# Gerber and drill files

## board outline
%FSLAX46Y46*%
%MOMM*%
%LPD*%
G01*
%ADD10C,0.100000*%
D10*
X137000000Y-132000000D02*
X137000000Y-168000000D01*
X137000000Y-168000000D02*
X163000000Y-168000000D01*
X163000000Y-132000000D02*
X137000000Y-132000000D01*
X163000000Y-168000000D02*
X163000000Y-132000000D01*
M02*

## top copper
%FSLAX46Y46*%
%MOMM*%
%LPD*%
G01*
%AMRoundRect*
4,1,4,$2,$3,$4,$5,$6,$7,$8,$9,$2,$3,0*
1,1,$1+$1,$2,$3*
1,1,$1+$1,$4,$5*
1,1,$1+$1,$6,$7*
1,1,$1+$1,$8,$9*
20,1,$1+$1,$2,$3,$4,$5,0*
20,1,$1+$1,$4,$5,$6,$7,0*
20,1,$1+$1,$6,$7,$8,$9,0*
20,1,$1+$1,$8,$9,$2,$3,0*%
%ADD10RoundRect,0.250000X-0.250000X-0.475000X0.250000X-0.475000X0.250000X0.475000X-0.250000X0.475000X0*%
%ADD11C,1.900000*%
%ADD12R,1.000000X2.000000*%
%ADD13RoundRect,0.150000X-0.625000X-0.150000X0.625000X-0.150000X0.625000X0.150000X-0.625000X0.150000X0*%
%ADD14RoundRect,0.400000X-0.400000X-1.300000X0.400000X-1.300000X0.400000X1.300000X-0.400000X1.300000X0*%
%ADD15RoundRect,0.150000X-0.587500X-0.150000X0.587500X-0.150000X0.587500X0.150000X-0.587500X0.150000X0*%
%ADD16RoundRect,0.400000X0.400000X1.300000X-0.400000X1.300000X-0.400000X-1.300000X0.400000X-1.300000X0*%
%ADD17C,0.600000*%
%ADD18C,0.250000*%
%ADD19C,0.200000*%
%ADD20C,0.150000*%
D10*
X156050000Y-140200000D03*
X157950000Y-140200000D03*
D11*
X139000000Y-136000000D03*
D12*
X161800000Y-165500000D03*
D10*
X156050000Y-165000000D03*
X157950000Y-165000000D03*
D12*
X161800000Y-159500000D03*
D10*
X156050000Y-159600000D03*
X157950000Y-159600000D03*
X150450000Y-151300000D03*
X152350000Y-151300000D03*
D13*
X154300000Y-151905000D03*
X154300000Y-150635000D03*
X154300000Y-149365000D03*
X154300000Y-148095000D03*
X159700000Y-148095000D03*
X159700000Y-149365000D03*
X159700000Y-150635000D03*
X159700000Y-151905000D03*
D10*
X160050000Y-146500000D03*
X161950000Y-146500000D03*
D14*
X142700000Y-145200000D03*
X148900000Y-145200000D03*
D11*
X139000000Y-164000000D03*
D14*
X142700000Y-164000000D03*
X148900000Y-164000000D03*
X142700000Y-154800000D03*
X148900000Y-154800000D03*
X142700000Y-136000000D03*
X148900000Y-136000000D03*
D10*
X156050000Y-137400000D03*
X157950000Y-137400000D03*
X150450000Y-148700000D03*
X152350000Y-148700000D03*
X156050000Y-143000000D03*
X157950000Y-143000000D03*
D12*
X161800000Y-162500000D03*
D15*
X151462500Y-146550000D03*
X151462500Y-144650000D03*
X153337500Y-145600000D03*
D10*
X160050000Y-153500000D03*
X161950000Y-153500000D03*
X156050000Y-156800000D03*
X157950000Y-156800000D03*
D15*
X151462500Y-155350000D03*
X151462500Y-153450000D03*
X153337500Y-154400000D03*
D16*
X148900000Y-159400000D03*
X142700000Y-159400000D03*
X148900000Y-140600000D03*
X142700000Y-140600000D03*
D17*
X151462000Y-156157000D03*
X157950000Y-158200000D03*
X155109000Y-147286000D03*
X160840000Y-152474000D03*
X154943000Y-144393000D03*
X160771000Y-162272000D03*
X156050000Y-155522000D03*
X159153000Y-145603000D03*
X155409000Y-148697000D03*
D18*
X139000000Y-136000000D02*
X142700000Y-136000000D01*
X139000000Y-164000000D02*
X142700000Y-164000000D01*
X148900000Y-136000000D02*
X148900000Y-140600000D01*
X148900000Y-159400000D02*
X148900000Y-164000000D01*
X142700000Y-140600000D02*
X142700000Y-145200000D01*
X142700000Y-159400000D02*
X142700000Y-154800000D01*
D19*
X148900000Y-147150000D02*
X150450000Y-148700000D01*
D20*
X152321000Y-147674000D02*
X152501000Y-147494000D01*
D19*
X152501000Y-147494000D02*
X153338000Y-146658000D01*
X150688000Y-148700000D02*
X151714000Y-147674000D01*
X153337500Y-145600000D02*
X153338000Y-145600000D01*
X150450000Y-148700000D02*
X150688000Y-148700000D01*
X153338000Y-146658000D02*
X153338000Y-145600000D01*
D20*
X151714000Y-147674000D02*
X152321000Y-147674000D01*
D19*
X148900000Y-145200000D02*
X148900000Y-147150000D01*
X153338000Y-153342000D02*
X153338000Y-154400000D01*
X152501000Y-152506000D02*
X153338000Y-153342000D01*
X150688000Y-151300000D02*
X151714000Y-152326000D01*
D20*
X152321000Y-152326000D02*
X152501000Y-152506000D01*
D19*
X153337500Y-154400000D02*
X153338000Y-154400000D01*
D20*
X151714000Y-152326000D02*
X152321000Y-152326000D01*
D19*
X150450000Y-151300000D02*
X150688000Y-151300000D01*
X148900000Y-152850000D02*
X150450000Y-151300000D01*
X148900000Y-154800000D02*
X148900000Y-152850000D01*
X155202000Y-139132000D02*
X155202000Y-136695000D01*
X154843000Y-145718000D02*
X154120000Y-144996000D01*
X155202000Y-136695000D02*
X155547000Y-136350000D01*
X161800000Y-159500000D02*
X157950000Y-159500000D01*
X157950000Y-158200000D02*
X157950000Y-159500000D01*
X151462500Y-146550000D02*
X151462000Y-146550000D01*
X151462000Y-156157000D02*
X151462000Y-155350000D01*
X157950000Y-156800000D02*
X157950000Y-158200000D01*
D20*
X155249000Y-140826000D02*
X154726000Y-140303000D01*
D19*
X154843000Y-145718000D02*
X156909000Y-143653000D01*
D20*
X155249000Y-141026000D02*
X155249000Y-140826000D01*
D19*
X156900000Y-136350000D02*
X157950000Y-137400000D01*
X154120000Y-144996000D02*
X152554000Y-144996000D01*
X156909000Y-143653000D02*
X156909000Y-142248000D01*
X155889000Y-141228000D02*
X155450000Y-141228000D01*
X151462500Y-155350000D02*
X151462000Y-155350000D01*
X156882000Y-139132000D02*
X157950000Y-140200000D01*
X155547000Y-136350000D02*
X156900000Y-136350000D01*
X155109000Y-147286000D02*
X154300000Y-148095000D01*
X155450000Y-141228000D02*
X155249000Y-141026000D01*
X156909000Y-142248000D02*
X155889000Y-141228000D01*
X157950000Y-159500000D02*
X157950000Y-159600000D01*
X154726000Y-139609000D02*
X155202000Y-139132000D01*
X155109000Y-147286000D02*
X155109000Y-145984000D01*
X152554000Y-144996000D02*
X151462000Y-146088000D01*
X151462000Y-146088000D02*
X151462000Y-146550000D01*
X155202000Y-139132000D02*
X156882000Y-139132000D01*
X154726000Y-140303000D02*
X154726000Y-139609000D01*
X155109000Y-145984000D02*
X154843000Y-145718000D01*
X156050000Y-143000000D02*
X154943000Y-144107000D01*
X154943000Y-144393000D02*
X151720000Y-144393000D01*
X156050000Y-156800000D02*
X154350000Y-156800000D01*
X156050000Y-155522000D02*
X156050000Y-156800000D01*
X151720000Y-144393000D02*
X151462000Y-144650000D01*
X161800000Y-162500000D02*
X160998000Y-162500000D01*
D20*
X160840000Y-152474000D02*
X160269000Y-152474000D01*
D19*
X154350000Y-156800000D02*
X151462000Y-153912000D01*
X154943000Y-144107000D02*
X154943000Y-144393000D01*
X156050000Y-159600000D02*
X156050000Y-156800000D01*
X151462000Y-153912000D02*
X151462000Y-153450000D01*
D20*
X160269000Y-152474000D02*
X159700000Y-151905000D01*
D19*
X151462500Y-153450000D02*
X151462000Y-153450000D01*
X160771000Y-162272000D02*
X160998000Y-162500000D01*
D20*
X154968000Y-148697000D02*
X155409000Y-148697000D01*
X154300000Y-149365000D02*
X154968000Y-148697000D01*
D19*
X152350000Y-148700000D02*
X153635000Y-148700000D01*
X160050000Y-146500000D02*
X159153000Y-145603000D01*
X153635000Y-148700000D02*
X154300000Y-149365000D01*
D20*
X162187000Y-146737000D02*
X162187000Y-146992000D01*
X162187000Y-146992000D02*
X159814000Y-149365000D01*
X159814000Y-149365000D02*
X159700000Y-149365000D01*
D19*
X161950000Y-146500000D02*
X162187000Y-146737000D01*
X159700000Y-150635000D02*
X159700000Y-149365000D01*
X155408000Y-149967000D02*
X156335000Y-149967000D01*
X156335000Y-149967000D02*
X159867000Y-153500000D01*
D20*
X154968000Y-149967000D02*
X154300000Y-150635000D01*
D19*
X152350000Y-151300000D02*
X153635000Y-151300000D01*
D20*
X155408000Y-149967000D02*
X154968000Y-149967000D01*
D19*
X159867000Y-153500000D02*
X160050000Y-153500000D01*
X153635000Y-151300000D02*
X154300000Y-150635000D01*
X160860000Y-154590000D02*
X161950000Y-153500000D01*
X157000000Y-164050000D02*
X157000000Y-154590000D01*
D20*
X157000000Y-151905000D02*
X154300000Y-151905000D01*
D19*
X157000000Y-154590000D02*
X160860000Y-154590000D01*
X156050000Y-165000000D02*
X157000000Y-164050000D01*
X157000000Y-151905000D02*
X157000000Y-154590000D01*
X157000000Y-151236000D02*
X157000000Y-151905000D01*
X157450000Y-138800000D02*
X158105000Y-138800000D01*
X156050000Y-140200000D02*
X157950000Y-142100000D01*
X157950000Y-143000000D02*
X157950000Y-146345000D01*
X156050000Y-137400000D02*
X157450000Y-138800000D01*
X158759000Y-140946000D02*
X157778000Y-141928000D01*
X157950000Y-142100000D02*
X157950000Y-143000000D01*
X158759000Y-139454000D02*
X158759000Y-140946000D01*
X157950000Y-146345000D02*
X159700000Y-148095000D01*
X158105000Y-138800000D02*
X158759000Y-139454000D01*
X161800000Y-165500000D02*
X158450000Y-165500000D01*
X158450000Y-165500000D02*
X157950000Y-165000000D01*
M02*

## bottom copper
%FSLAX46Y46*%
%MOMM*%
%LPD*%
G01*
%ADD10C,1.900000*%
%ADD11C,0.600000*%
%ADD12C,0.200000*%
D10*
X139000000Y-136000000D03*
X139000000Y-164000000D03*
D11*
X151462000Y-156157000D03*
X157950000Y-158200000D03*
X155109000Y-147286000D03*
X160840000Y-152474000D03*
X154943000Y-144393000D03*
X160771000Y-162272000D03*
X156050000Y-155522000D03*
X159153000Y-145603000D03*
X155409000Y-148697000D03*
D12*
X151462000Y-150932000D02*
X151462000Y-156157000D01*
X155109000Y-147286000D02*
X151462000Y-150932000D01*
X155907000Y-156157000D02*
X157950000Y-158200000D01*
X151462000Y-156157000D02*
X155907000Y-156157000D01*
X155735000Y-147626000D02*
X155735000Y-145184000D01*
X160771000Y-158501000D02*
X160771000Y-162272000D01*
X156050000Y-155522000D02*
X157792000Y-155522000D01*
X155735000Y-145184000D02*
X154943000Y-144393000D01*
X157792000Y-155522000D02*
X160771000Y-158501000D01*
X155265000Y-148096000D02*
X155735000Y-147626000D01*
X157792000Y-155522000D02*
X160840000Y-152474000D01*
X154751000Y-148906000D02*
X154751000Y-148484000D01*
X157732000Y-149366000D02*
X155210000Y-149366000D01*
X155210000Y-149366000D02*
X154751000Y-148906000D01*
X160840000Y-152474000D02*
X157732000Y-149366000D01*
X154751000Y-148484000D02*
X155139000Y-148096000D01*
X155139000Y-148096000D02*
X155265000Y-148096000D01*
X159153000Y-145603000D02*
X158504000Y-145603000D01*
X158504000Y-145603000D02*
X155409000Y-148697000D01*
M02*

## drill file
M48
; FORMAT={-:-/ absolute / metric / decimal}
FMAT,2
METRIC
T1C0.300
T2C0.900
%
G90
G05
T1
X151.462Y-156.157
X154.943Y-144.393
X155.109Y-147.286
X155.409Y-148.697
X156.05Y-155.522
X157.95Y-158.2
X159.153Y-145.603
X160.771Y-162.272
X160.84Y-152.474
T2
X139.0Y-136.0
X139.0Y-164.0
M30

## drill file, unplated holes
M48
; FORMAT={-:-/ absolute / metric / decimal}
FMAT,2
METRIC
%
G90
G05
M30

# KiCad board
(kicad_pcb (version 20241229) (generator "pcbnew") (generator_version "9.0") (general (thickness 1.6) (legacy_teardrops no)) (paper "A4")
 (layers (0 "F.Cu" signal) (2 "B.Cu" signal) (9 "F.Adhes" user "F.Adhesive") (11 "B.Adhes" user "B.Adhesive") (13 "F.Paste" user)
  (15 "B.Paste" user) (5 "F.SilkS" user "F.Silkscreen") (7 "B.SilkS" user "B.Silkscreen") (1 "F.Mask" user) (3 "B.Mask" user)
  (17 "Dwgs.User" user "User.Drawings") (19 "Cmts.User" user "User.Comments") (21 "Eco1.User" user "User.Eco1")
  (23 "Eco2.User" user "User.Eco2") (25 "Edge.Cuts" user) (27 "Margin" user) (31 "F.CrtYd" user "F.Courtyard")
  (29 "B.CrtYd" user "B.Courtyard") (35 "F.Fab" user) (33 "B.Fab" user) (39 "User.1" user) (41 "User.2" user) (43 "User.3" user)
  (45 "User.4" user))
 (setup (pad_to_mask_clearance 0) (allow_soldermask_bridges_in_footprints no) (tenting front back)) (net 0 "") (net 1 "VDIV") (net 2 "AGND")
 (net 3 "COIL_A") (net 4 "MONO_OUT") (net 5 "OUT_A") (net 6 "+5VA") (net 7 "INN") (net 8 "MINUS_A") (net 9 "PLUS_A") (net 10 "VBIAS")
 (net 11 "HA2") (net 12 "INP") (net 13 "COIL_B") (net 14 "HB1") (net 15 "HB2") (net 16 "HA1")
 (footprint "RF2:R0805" (layer "F.Cu") (at 157 140.2)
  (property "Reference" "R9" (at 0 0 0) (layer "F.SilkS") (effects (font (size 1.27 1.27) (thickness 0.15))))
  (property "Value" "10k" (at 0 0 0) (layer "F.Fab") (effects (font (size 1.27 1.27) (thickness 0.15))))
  (pad "1" smd roundrect (at -0.95 0) (size 1 1.45) (layers "F.Cu" "F.Mask" "F.Paste") (roundrect_rratio 0.25) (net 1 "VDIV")
   (thermal_bridge_angle 45))
  (pad "2" smd roundrect (at 0.95 0) (size 1 1.45) (layers "F.Cu" "F.Mask" "F.Paste") (roundrect_rratio 0.25) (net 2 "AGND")
   (thermal_bridge_angle 45)))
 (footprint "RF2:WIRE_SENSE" (layer "F.Cu") (at 139 136)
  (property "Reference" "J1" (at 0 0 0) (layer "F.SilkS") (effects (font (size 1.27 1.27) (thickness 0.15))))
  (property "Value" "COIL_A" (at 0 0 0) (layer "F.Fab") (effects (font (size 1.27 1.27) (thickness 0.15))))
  (pad "1" thru_hole circle (at 0 0) (size 1.9 1.9) (drill 0.9) (layers "*.Cu" "*.Mask") (remove_unused_layers no) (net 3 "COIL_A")))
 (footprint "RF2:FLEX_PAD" (layer "F.Cu") (at 161.8 165.5)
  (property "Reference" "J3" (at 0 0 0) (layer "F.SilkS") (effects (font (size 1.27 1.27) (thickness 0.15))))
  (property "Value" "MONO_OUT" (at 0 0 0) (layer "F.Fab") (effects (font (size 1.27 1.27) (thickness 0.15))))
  (pad "1" smd rect (at 0 0) (size 1 2) (layers "F.Cu" "F.Mask" "F.Paste") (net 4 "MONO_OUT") (thermal_bridge_angle 45)))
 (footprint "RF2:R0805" (layer "F.Cu") (at 157 165)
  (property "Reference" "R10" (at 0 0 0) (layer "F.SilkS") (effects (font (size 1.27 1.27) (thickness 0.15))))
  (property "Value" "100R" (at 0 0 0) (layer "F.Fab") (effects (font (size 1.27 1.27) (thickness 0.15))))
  (pad "1" smd roundrect (at -0.95 0) (size 1 1.45) (layers "F.Cu" "F.Mask" "F.Paste") (roundrect_rratio 0.25) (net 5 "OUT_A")
   (thermal_bridge_angle 45))
  (pad "2" smd roundrect (at 0.95 0) (size 1 1.45) (layers "F.Cu" "F.Mask" "F.Paste") (roundrect_rratio 0.25) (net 4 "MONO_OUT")
   (thermal_bridge_angle 45)))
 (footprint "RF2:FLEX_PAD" (layer "F.Cu") (at 161.8 159.5)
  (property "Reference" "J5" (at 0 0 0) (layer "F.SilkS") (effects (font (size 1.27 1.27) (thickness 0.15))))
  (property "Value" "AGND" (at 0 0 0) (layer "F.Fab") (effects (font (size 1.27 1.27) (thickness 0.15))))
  (pad "1" smd rect (at 0 0) (size 1 2) (layers "F.Cu" "F.Mask" "F.Paste") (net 2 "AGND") (thermal_bridge_angle 45)))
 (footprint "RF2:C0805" (layer "F.Cu") (at 157 159.6)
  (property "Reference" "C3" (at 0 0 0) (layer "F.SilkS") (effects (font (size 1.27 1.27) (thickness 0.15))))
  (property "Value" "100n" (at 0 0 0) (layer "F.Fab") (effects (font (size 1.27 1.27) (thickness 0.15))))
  (pad "1" smd roundrect (at -0.95 0) (size 1 1.45) (layers "F.Cu" "F.Mask" "F.Paste") (roundrect_rratio 0.25) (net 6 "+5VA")
   (thermal_bridge_angle 45))
  (pad "2" smd roundrect (at 0.95 0) (size 1 1.45) (layers "F.Cu" "F.Mask" "F.Paste") (roundrect_rratio 0.25) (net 2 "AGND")
   (thermal_bridge_angle 45)))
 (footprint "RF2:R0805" (layer "F.Cu") (at 151.4 151.3)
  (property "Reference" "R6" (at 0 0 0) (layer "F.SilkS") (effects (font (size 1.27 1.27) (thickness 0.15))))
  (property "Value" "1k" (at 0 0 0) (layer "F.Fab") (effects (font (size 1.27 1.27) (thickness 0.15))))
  (pad "1" smd roundrect (at -0.95 0) (size 1 1.45) (layers "F.Cu" "F.Mask" "F.Paste") (roundrect_rratio 0.25) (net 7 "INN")
   (thermal_bridge_angle 45))
  (pad "2" smd roundrect (at 0.95 0) (size 1 1.45) (layers "F.Cu" "F.Mask" "F.Paste") (roundrect_rratio 0.25) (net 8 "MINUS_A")
   (thermal_bridge_angle 45)))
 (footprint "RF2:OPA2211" (layer "F.Cu") (at 157 150)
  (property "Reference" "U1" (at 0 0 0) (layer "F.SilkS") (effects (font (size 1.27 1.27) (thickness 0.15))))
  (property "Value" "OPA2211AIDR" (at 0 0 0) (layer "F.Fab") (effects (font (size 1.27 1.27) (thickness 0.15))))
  (pad "1" smd roundrect (at -2.7 1.905) (size 1.55 0.6) (layers "F.Cu" "F.Mask" "F.Paste") (roundrect_rratio 0.25) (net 5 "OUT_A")
   (thermal_bridge_angle 45))
  (pad "2" smd roundrect (at -2.7 0.635) (size 1.55 0.6) (layers "F.Cu" "F.Mask" "F.Paste") (roundrect_rratio 0.25) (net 8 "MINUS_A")
   (thermal_bridge_angle 45))
  (pad "3" smd roundrect (at -2.7 -0.635) (size 1.55 0.6) (layers "F.Cu" "F.Mask" "F.Paste") (roundrect_rratio 0.25) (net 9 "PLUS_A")
   (thermal_bridge_angle 45))
  (pad "4" smd roundrect (at -2.7 -1.905) (size 1.55 0.6) (layers "F.Cu" "F.Mask" "F.Paste") (roundrect_rratio 0.25) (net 2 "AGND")
   (thermal_bridge_angle 45))
  (pad "5" smd roundrect (at 2.7 -1.905) (size 1.55 0.6) (layers "F.Cu" "F.Mask" "F.Paste") (roundrect_rratio 0.25) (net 1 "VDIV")
   (thermal_bridge_angle 45))
  (pad "6" smd roundrect (at 2.7 -0.635) (size 1.55 0.6) (layers "F.Cu" "F.Mask" "F.Paste") (roundrect_rratio 0.25) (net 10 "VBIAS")
   (thermal_bridge_angle 45))
  (pad "7" smd roundrect (at 2.7 0.635) (size 1.55 0.6) (layers "F.Cu" "F.Mask" "F.Paste") (roundrect_rratio 0.25) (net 10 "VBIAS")
   (thermal_bridge_angle 45))
  (pad "8" smd roundrect (at 2.7 1.905) (size 1.55 0.6) (layers "F.Cu" "F.Mask" "F.Paste") (roundrect_rratio 0.25) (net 6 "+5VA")
   (thermal_bridge_angle 45)))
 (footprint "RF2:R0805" (layer "F.Cu") (at 161 146.5)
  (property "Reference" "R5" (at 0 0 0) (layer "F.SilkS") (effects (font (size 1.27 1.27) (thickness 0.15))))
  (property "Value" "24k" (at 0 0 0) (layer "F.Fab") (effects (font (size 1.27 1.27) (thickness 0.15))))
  (pad "1" smd roundrect (at -0.95 0) (size 1 1.45) (layers "F.Cu" "F.Mask" "F.Paste") (roundrect_rratio 0.25) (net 9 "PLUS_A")
   (thermal_bridge_angle 45))
  (pad "2" smd roundrect (at 0.95 0) (size 1 1.45) (layers "F.Cu" "F.Mask" "F.Paste") (roundrect_rratio 0.25) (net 10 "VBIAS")
   (thermal_bridge_angle 45)))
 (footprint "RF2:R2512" (layer "F.Cu") (at 145.8 145.2)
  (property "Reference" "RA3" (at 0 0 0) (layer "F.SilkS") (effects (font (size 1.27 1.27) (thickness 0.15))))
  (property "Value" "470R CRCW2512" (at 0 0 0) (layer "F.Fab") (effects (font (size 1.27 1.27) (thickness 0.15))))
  (pad "1" smd roundrect (at -3.1 0) (size 1.6 3.4) (layers "F.Cu" "F.Mask" "F.Paste") (roundrect_rratio 0.25) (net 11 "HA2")
   (thermal_bridge_angle 45))
  (pad "2" smd roundrect (at 3.1 0) (size 1.6 3.4) (layers "F.Cu" "F.Mask" "F.Paste") (roundrect_rratio 0.25) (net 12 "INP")
   (thermal_bridge_angle 45)))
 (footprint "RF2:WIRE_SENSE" (layer "F.Cu") (at 139 164)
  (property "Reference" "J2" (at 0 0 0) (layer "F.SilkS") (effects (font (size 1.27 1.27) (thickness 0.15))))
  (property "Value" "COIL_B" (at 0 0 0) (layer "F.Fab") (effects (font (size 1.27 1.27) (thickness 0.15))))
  (pad "1" thru_hole circle (at 0 0) (size 1.9 1.9) (drill 0.9) (layers "*.Cu" "*.Mask") (remove_unused_layers no) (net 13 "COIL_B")))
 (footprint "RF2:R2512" (layer "F.Cu") (at 145.8 164)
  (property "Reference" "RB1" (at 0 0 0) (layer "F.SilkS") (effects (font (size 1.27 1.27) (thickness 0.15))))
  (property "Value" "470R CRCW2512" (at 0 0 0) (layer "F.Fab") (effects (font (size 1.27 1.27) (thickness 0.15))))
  (pad "1" smd roundrect (at -3.1 0) (size 1.6 3.4) (layers "F.Cu" "F.Mask" "F.Paste") (roundrect_rratio 0.25) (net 13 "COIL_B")
   (thermal_bridge_angle 45))
  (pad "2" smd roundrect (at 3.1 0) (size 1.6 3.4) (layers "F.Cu" "F.Mask" "F.Paste") (roundrect_rratio 0.25) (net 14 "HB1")
   (thermal_bridge_angle 45)))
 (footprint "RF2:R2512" (layer "F.Cu") (at 145.8 154.8)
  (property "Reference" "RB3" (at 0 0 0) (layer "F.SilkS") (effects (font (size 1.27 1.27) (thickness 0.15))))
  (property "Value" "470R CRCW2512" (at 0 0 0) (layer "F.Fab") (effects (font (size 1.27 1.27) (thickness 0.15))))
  (pad "1" smd roundrect (at -3.1 0) (size 1.6 3.4) (layers "F.Cu" "F.Mask" "F.Paste") (roundrect_rratio 0.25) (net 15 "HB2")
   (thermal_bridge_angle 45))
  (pad "2" smd roundrect (at 3.1 0) (size 1.6 3.4) (layers "F.Cu" "F.Mask" "F.Paste") (roundrect_rratio 0.25) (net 7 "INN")
   (thermal_bridge_angle 45)))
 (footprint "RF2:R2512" (layer "F.Cu") (at 145.8 136)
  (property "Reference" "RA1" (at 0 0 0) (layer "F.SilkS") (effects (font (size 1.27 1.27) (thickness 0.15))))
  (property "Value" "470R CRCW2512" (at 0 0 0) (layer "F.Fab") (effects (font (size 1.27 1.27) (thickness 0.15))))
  (pad "1" smd roundrect (at -3.1 0) (size 1.6 3.4) (layers "F.Cu" "F.Mask" "F.Paste") (roundrect_rratio 0.25) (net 3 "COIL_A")
   (thermal_bridge_angle 45))
  (pad "2" smd roundrect (at 3.1 0) (size 1.6 3.4) (layers "F.Cu" "F.Mask" "F.Paste") (roundrect_rratio 0.25) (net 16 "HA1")
   (thermal_bridge_angle 45)))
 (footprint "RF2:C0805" (layer "F.Cu") (at 157 137.4)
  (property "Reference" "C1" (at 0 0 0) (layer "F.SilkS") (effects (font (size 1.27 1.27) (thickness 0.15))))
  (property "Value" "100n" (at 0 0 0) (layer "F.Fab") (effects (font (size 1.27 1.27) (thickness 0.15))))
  (pad "1" smd roundrect (at -0.95 0) (size 1 1.45) (layers "F.Cu" "F.Mask" "F.Paste") (roundrect_rratio 0.25) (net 1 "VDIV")
   (thermal_bridge_angle 45))
  (pad "2" smd roundrect (at 0.95 0) (size 1 1.45) (layers "F.Cu" "F.Mask" "F.Paste") (roundrect_rratio 0.25) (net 2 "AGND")
   (thermal_bridge_angle 45)))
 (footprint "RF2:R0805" (layer "F.Cu") (at 151.4 148.7)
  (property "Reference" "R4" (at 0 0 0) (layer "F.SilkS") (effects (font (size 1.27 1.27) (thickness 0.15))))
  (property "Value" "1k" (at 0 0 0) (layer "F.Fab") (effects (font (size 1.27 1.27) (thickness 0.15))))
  (pad "1" smd roundrect (at -0.95 0) (size 1 1.45) (layers "F.Cu" "F.Mask" "F.Paste") (roundrect_rratio 0.25) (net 12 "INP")
   (thermal_bridge_angle 45))
  (pad "2" smd roundrect (at 0.95 0) (size 1 1.45) (layers "F.Cu" "F.Mask" "F.Paste") (roundrect_rratio 0.25) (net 9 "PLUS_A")
   (thermal_bridge_angle 45)))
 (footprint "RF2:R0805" (layer "F.Cu") (at 157 143)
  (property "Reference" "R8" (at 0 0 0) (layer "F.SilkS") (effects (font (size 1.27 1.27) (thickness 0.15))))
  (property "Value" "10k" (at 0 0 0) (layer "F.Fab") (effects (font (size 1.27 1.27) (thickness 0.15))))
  (pad "1" smd roundrect (at -0.95 0) (size 1 1.45) (layers "F.Cu" "F.Mask" "F.Paste") (roundrect_rratio 0.25) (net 6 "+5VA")
   (thermal_bridge_angle 45))
  (pad "2" smd roundrect (at 0.95 0) (size 1 1.45) (layers "F.Cu" "F.Mask" "F.Paste") (roundrect_rratio 0.25) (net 1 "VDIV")
   (thermal_bridge_angle 45)))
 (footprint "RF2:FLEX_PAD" (layer "F.Cu") (at 161.8 162.5)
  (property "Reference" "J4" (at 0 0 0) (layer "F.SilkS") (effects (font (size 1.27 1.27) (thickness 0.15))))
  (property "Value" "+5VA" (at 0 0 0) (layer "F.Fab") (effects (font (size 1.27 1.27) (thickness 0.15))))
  (pad "1" smd rect (at 0 0) (size 1 2) (layers "F.Cu" "F.Mask" "F.Paste") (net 6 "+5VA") (thermal_bridge_angle 45)))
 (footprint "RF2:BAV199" (layer "F.Cu") (at 152.4 145.6)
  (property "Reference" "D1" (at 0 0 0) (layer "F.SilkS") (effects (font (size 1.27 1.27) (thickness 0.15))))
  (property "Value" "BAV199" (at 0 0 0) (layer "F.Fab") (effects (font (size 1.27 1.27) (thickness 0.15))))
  (pad "1" smd roundrect (at -0.9375 0.95) (size 1.475 0.6) (layers "F.Cu" "F.Mask" "F.Paste") (roundrect_rratio 0.25) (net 2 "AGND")
   (thermal_bridge_angle 45))
  (pad "2" smd roundrect (at -0.9375 -0.95) (size 1.475 0.6) (layers "F.Cu" "F.Mask" "F.Paste") (roundrect_rratio 0.25) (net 6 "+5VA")
   (thermal_bridge_angle 45))
  (pad "3" smd roundrect (at 0.9375 0) (size 1.475 0.6) (layers "F.Cu" "F.Mask" "F.Paste") (roundrect_rratio 0.25) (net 12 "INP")
   (thermal_bridge_angle 45)))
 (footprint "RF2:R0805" (layer "F.Cu") (at 161 153.5)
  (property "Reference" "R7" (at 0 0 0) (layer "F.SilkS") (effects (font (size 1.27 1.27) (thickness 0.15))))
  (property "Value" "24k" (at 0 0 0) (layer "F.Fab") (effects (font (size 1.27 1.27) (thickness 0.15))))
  (pad "1" smd roundrect (at -0.95 0) (size 1 1.45) (layers "F.Cu" "F.Mask" "F.Paste") (roundrect_rratio 0.25) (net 8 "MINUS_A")
   (thermal_bridge_angle 45))
  (pad "2" smd roundrect (at 0.95 0) (size 1 1.45) (layers "F.Cu" "F.Mask" "F.Paste") (roundrect_rratio 0.25) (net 5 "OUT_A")
   (thermal_bridge_angle 45)))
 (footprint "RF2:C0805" (layer "F.Cu") (at 157 156.8)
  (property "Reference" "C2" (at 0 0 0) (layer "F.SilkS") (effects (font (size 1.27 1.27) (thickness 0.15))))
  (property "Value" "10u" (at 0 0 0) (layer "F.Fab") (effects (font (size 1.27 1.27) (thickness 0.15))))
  (pad "1" smd roundrect (at -0.95 0) (size 1 1.45) (layers "F.Cu" "F.Mask" "F.Paste") (roundrect_rratio 0.25) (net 6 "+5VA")
   (thermal_bridge_angle 45))
  (pad "2" smd roundrect (at 0.95 0) (size 1 1.45) (layers "F.Cu" "F.Mask" "F.Paste") (roundrect_rratio 0.25) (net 2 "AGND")
   (thermal_bridge_angle 45)))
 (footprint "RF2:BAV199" (layer "F.Cu") (at 152.4 154.4)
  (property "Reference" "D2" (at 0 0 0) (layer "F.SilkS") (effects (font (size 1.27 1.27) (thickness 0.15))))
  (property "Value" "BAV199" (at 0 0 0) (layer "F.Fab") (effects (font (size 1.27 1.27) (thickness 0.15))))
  (pad "1" smd roundrect (at -0.9375 0.95) (size 1.475 0.6) (layers "F.Cu" "F.Mask" "F.Paste") (roundrect_rratio 0.25) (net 2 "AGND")
   (thermal_bridge_angle 45))
  (pad "2" smd roundrect (at -0.9375 -0.95) (size 1.475 0.6) (layers "F.Cu" "F.Mask" "F.Paste") (roundrect_rratio 0.25) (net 6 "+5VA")
   (thermal_bridge_angle 45))
  (pad "3" smd roundrect (at 0.9375 0) (size 1.475 0.6) (layers "F.Cu" "F.Mask" "F.Paste") (roundrect_rratio 0.25) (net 7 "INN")
   (thermal_bridge_angle 45)))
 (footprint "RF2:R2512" (layer "F.Cu") (at 145.8 159.4 180)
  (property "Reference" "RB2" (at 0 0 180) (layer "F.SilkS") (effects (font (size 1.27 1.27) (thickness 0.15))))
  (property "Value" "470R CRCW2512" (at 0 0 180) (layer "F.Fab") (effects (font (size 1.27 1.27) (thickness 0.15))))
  (pad "1" smd roundrect (at -3.1 0 180) (size 1.6 3.4) (layers "F.Cu" "F.Mask" "F.Paste") (roundrect_rratio 0.25) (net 14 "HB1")
   (thermal_bridge_angle 45))
  (pad "2" smd roundrect (at 3.1 0 180) (size 1.6 3.4) (layers "F.Cu" "F.Mask" "F.Paste") (roundrect_rratio 0.25) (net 15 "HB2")
   (thermal_bridge_angle 45)))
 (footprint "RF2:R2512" (layer "F.Cu") (at 145.8 140.6 180)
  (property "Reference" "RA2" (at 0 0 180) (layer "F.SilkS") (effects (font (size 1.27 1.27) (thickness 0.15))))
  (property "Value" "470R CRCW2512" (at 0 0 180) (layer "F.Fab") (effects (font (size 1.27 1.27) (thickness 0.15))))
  (pad "1" smd roundrect (at -3.1 0 180) (size 1.6 3.4) (layers "F.Cu" "F.Mask" "F.Paste") (roundrect_rratio 0.25) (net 16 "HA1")
   (thermal_bridge_angle 45))
  (pad "2" smd roundrect (at 3.1 0 180) (size 1.6 3.4) (layers "F.Cu" "F.Mask" "F.Paste") (roundrect_rratio 0.25) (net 11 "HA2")
   (thermal_bridge_angle 45)))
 (gr_line (start 137 132) (end 137 168) (stroke (width 0.1) (type default)) (layer "Edge.Cuts"))
 (gr_line (start 137 168) (end 163 168) (stroke (width 0.1) (type default)) (layer "Edge.Cuts"))
 (gr_line (start 163 132) (end 137 132) (stroke (width 0.1) (type default)) (layer "Edge.Cuts"))
 (gr_line (start 163 168) (end 163 132) (stroke (width 0.1) (type default)) (layer "Edge.Cuts"))
 (segment (start 139 136) (end 142.7 136) (width 0.25) (layer "F.Cu") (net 3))
 (segment (start 139 164) (end 142.7 164) (width 0.25) (layer "F.Cu") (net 13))
 (segment (start 148.9 136) (end 148.9 140.6) (width 0.25) (layer "F.Cu") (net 16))
 (segment (start 148.9 159.4) (end 148.9 164) (width 0.25) (layer "F.Cu") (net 14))
 (segment (start 142.7 140.6) (end 142.7 145.2) (width 0.25) (layer "F.Cu") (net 11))
 (segment (start 142.7 159.4) (end 142.7 154.8) (width 0.25) (layer "F.Cu") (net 15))
 (segment (start 148.9 147.15) (end 150.45 148.7) (width 0.2) (layer "F.Cu") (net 12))
 (segment (start 152.321 147.674) (end 152.501 147.494) (width 0.15) (layer "F.Cu") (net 12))
 (segment (start 152.501 147.494) (end 153.338 146.658) (width 0.2) (layer "F.Cu") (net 12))
 (segment (start 150.688 148.7) (end 151.714 147.674) (width 0.2) (layer "F.Cu") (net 12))
 (segment (start 153.3375 145.6) (end 153.338 145.6) (width 0.2) (layer "F.Cu") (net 12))
 (segment (start 150.45 148.7) (end 150.688 148.7) (width 0.2) (layer "F.Cu") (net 12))
 (segment (start 153.338 146.658) (end 153.338 145.6) (width 0.2) (layer "F.Cu") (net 12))
 (segment (start 151.714 147.674) (end 152.321 147.674) (width 0.15) (layer "F.Cu") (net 12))
 (segment (start 148.9 145.2) (end 148.9 147.15) (width 0.2) (layer "F.Cu") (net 12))
 (segment (start 153.338 153.342) (end 153.338 154.4) (width 0.2) (layer "F.Cu") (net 7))
 (segment (start 152.501 152.506) (end 153.338 153.342) (width 0.2) (layer "F.Cu") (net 7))
 (segment (start 150.688 151.3) (end 151.714 152.326) (width 0.2) (layer "F.Cu") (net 7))
 (segment (start 152.321 152.326) (end 152.501 152.506) (width 0.15) (layer "F.Cu") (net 7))
 (segment (start 153.3375 154.4) (end 153.338 154.4) (width 0.2) (layer "F.Cu") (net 7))
 (segment (start 151.714 152.326) (end 152.321 152.326) (width 0.15) (layer "F.Cu") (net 7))
 (segment (start 150.45 151.3) (end 150.688 151.3) (width 0.2) (layer "F.Cu") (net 7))
 (segment (start 148.9 152.85) (end 150.45 151.3) (width 0.2) (layer "F.Cu") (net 7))
 (segment (start 148.9 154.8) (end 148.9 152.85) (width 0.2) (layer "F.Cu") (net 7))
 (segment (start 155.202 139.132) (end 155.202 136.695) (width 0.2) (layer "F.Cu") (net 2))
 (segment (start 154.843 145.718) (end 154.12 144.996) (width 0.2) (layer "F.Cu") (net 2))
 (segment (start 155.202 136.695) (end 155.547 136.35) (width 0.2) (layer "F.Cu") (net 2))
 (segment (start 161.8 159.5) (end 157.95 159.5) (width 0.2) (layer "F.Cu") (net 2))
 (segment (start 157.95 158.2) (end 157.95 159.5) (width 0.2) (layer "F.Cu") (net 2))
 (segment (start 151.4625 146.55) (end 151.462 146.55) (width 0.2) (layer "F.Cu") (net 2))
 (segment (start 151.462 156.157) (end 151.462 155.35) (width 0.2) (layer "F.Cu") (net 2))
 (segment (start 157.95 156.8) (end 157.95 158.2) (width 0.2) (layer "F.Cu") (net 2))
 (segment (start 155.249 140.826) (end 154.726 140.303) (width 0.15) (layer "F.Cu") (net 2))
 (segment (start 154.843 145.718) (end 156.909 143.653) (width 0.2) (layer "F.Cu") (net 2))
 (segment (start 155.249 141.026) (end 155.249 140.826) (width 0.15) (layer "F.Cu") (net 2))
 (segment (start 156.9 136.35) (end 157.95 137.4) (width 0.2) (layer "F.Cu") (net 2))
 (segment (start 154.12 144.996) (end 152.554 144.996) (width 0.2) (layer "F.Cu") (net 2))
 (segment (start 156.909 143.653) (end 156.909 142.248) (width 0.2) (layer "F.Cu") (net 2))
 (segment (start 155.889 141.228) (end 155.45 141.228) (width 0.2) (layer "F.Cu") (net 2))
 (segment (start 151.4625 155.35) (end 151.462 155.35) (width 0.2) (layer "F.Cu") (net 2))
 (segment (start 156.882 139.132) (end 157.95 140.2) (width 0.2) (layer "F.Cu") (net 2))
 (segment (start 155.547 136.35) (end 156.9 136.35) (width 0.2) (layer "F.Cu") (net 2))
 (segment (start 155.109 147.286) (end 154.3 148.095) (width 0.2) (layer "F.Cu") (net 2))
 (segment (start 155.45 141.228) (end 155.249 141.026) (width 0.2) (layer "F.Cu") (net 2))
 (segment (start 156.909 142.248) (end 155.889 141.228) (width 0.2) (layer "F.Cu") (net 2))
 (segment (start 157.95 159.5) (end 157.95 159.6) (width 0.2) (layer "F.Cu") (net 2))
 (segment (start 154.726 139.609) (end 155.202 139.132) (width 0.2) (layer "F.Cu") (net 2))
 (segment (start 155.109 147.286) (end 155.109 145.984) (width 0.2) (layer "F.Cu") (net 2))
 (segment (start 152.554 144.996) (end 151.462 146.088) (width 0.2) (layer "F.Cu") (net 2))
 (segment (start 151.462 146.088) (end 151.462 146.55) (width 0.2) (layer "F.Cu") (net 2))
 (segment (start 155.202 139.132) (end 156.882 139.132) (width 0.2) (layer "F.Cu") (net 2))
 (segment (start 154.726 140.303) (end 154.726 139.609) (width 0.2) (layer "F.Cu") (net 2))
 (segment (start 155.109 145.984) (end 154.843 145.718) (width 0.2) (layer "F.Cu") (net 2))
 (via (at 151.462 156.157) (size 0.6) (drill 0.3) (layers "F.Cu" "B.Cu") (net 2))
 (via (at 157.95 158.2) (size 0.6) (drill 0.3) (layers "F.Cu" "B.Cu") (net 2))
 (via (at 155.109 147.286) (size 0.6) (drill 0.3) (layers "F.Cu" "B.Cu") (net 2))
 (segment (start 151.462 150.932) (end 151.462 156.157) (width 0.2) (layer "B.Cu") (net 2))
 (segment (start 155.109 147.286) (end 151.462 150.932) (width 0.2) (layer "B.Cu") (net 2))
 (segment (start 155.907 156.157) (end 157.95 158.2) (width 0.2) (layer "B.Cu") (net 2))
 (segment (start 151.462 156.157) (end 155.907 156.157) (width 0.2) (layer "B.Cu") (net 2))
 (segment (start 156.05 143) (end 154.943 144.107) (width 0.2) (layer "F.Cu") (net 6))
 (segment (start 154.943 144.393) (end 151.72 144.393) (width 0.2) (layer "F.Cu") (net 6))
 (segment (start 156.05 156.8) (end 154.35 156.8) (width 0.2) (layer "F.Cu") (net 6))
 (segment (start 156.05 155.522) (end 156.05 156.8) (width 0.2) (layer "F.Cu") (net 6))
 (segment (start 151.72 144.393) (end 151.462 144.65) (width 0.2) (layer "F.Cu") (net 6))
 (segment (start 161.8 162.5) (end 160.998 162.5) (width 0.2) (layer "F.Cu") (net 6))
 (segment (start 160.84 152.474) (end 160.269 152.474) (width 0.15) (layer "F.Cu") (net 6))
 (segment (start 154.35 156.8) (end 151.462 153.912) (width 0.2) (layer "F.Cu") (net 6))
 (segment (start 154.943 144.107) (end 154.943 144.393) (width 0.2) (layer "F.Cu") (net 6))
 (segment (start 156.05 159.6) (end 156.05 156.8) (width 0.2) (layer "F.Cu") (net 6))
 (segment (start 151.462 153.912) (end 151.462 153.45) (width 0.2) (layer "F.Cu") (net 6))
 (segment (start 160.269 152.474) (end 159.7 151.905) (width 0.15) (layer "F.Cu") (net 6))
 (segment (start 151.4625 153.45) (end 151.462 153.45) (width 0.2) (layer "F.Cu") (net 6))
 (segment (start 160.771 162.272) (end 160.998 162.5) (width 0.2) (layer "F.Cu") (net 6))
 (via (at 160.84 152.474) (size 0.6) (drill 0.3) (layers "F.Cu" "B.Cu") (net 6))
 (via (at 154.943 144.393) (size 0.6) (drill 0.3) (layers "F.Cu" "B.Cu") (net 6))
 (via (at 160.771 162.272) (size 0.6) (drill 0.3) (layers "F.Cu" "B.Cu") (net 6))
 (via (at 156.05 155.522) (size 0.6) (drill 0.3) (layers "F.Cu" "B.Cu") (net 6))
 (segment (start 155.735 147.626) (end 155.735 145.184) (width 0.2) (layer "B.Cu") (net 6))
 (segment (start 160.771 158.501) (end 160.771 162.272) (width 0.2) (layer "B.Cu") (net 6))
 (segment (start 156.05 155.522) (end 157.792 155.522) (width 0.2) (layer "B.Cu") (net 6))
 (segment (start 155.735 145.184) (end 154.943 144.393) (width 0.2) (layer "B.Cu") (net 6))
 (segment (start 157.792 155.522) (end 160.771 158.501) (width 0.2) (layer "B.Cu") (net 6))
 (segment (start 155.265 148.096) (end 155.735 147.626) (width 0.2) (layer "B.Cu") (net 6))
 (segment (start 157.792 155.522) (end 160.84 152.474) (width 0.2) (layer "B.Cu") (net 6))
 (segment (start 154.751 148.906) (end 154.751 148.484) (width 0.2) (layer "B.Cu") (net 6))
 (segment (start 157.732 149.366) (end 155.21 149.366) (width 0.2) (layer "B.Cu") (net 6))
 (segment (start 155.21 149.366) (end 154.751 148.906) (width 0.2) (layer "B.Cu") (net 6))
 (segment (start 160.84 152.474) (end 157.732 149.366) (width 0.2) (layer "B.Cu") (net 6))
 (segment (start 154.751 148.484) (end 155.139 148.096) (width 0.2) (layer "B.Cu") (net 6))
 (segment (start 155.139 148.096) (end 155.265 148.096) (width 0.2) (layer "B.Cu") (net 6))
 (segment (start 154.968 148.697) (end 155.409 148.697) (width 0.15) (layer "F.Cu") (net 9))
 (segment (start 154.3 149.365) (end 154.968 148.697) (width 0.15) (layer "F.Cu") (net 9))
 (segment (start 152.35 148.7) (end 153.635 148.7) (width 0.2) (layer "F.Cu") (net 9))
 (segment (start 160.05 146.5) (end 159.153 145.603) (width 0.2) (layer "F.Cu") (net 9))
 (segment (start 153.635 148.7) (end 154.3 149.365) (width 0.2) (layer "F.Cu") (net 9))
 (via (at 159.153 145.603) (size 0.6) (drill 0.3) (layers "F.Cu" "B.Cu") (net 9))
 (via (at 155.409 148.697) (size 0.6) (drill 0.3) (layers "F.Cu" "B.Cu") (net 9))
 (segment (start 159.153 145.603) (end 158.504 145.603) (width 0.2) (layer "B.Cu") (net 9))
 (segment (start 158.504 145.603) (end 155.409 148.697) (width 0.2) (layer "B.Cu") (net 9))
 (segment (start 162.187 146.737) (end 162.187 146.992) (width 0.15) (layer "F.Cu") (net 10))
 (segment (start 162.187 146.992) (end 159.814 149.365) (width 0.15) (layer "F.Cu") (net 10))
 (segment (start 159.814 149.365) (end 159.7 149.365) (width 0.15) (layer "F.Cu") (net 10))
 (segment (start 161.95 146.5) (end 162.187 146.737) (width 0.2) (layer "F.Cu") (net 10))
 (segment (start 159.7 150.635) (end 159.7 149.365) (width 0.2) (layer "F.Cu") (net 10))
 (segment (start 155.408 149.967) (end 156.335 149.967) (width 0.2) (layer "F.Cu") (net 8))
 (segment (start 156.335 149.967) (end 159.867 153.5) (width 0.2) (layer "F.Cu") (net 8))
 (segment (start 154.968 149.967) (end 154.3 150.635) (width 0.15) (layer "F.Cu") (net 8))
 (segment (start 152.35 151.3) (end 153.635 151.3) (width 0.2) (layer "F.Cu") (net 8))
 (segment (start 155.408 149.967) (end 154.968 149.967) (width 0.15) (layer "F.Cu") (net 8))
 (segment (start 159.867 153.5) (end 160.05 153.5) (width 0.2) (layer "F.Cu") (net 8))
 (segment (start 153.635 151.3) (end 154.3 150.635) (width 0.2) (layer "F.Cu") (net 8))
 (segment (start 160.86 154.59) (end 161.95 153.5) (width 0.2) (layer "F.Cu") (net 5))
 (segment (start 157 164.05) (end 157 154.59) (width 0.2) (layer "F.Cu") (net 5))
 (segment (start 157 151.905) (end 154.3 151.905) (width 0.15) (layer "F.Cu") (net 5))
 (segment (start 157 154.59) (end 160.86 154.59) (width 0.2) (layer "F.Cu") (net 5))
 (segment (start 156.05 165) (end 157 164.05) (width 0.2) (layer "F.Cu") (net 5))
 (segment (start 157 151.905) (end 157 154.59) (width 0.2) (layer "F.Cu") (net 5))
 (segment (start 157 151.236) (end 157 151.905) (width 0.2) (layer "F.Cu") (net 5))
 (segment (start 157.45 138.8) (end 158.105 138.8) (width 0.2) (layer "F.Cu") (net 1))
 (segment (start 156.05 140.2) (end 157.95 142.1) (width 0.2) (layer "F.Cu") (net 1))
 (segment (start 157.95 143) (end 157.95 146.345) (width 0.2) (layer "F.Cu") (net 1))
 (segment (start 156.05 137.4) (end 157.45 138.8) (width 0.2) (layer "F.Cu") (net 1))
 (segment (start 158.759 140.946) (end 157.778 141.928) (width 0.2) (layer "F.Cu") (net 1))
 (segment (start 157.95 142.1) (end 157.95 143) (width 0.2) (layer "F.Cu") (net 1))
 (segment (start 158.759 139.454) (end 158.759 140.946) (width 0.2) (layer "F.Cu") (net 1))
 (segment (start 157.95 146.345) (end 159.7 148.095) (width 0.2) (layer "F.Cu") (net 1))
 (segment (start 158.105 138.8) (end 158.759 139.454) (width 0.2) (layer "F.Cu") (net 1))
 (segment (start 161.8 165.5) (end 158.45 165.5) (width 0.2) (layer "F.Cu") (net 4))
 (segment (start 158.45 165.5) (end 157.95 165) (width 0.2) (layer "F.Cu") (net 4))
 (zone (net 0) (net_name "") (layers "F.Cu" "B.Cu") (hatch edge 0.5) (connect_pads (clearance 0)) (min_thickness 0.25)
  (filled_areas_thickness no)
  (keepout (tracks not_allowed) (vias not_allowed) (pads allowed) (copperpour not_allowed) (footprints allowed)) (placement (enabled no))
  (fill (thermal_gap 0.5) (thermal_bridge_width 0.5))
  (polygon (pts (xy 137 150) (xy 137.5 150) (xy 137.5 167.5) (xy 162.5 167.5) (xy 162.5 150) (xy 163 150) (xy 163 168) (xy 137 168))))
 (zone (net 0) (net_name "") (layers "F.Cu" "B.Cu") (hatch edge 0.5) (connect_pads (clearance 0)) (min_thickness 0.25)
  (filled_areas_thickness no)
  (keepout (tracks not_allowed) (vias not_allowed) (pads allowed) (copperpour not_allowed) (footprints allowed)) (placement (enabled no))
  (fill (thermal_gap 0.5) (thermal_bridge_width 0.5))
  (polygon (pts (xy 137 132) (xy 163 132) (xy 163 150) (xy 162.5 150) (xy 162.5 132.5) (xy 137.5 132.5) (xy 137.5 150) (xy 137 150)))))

